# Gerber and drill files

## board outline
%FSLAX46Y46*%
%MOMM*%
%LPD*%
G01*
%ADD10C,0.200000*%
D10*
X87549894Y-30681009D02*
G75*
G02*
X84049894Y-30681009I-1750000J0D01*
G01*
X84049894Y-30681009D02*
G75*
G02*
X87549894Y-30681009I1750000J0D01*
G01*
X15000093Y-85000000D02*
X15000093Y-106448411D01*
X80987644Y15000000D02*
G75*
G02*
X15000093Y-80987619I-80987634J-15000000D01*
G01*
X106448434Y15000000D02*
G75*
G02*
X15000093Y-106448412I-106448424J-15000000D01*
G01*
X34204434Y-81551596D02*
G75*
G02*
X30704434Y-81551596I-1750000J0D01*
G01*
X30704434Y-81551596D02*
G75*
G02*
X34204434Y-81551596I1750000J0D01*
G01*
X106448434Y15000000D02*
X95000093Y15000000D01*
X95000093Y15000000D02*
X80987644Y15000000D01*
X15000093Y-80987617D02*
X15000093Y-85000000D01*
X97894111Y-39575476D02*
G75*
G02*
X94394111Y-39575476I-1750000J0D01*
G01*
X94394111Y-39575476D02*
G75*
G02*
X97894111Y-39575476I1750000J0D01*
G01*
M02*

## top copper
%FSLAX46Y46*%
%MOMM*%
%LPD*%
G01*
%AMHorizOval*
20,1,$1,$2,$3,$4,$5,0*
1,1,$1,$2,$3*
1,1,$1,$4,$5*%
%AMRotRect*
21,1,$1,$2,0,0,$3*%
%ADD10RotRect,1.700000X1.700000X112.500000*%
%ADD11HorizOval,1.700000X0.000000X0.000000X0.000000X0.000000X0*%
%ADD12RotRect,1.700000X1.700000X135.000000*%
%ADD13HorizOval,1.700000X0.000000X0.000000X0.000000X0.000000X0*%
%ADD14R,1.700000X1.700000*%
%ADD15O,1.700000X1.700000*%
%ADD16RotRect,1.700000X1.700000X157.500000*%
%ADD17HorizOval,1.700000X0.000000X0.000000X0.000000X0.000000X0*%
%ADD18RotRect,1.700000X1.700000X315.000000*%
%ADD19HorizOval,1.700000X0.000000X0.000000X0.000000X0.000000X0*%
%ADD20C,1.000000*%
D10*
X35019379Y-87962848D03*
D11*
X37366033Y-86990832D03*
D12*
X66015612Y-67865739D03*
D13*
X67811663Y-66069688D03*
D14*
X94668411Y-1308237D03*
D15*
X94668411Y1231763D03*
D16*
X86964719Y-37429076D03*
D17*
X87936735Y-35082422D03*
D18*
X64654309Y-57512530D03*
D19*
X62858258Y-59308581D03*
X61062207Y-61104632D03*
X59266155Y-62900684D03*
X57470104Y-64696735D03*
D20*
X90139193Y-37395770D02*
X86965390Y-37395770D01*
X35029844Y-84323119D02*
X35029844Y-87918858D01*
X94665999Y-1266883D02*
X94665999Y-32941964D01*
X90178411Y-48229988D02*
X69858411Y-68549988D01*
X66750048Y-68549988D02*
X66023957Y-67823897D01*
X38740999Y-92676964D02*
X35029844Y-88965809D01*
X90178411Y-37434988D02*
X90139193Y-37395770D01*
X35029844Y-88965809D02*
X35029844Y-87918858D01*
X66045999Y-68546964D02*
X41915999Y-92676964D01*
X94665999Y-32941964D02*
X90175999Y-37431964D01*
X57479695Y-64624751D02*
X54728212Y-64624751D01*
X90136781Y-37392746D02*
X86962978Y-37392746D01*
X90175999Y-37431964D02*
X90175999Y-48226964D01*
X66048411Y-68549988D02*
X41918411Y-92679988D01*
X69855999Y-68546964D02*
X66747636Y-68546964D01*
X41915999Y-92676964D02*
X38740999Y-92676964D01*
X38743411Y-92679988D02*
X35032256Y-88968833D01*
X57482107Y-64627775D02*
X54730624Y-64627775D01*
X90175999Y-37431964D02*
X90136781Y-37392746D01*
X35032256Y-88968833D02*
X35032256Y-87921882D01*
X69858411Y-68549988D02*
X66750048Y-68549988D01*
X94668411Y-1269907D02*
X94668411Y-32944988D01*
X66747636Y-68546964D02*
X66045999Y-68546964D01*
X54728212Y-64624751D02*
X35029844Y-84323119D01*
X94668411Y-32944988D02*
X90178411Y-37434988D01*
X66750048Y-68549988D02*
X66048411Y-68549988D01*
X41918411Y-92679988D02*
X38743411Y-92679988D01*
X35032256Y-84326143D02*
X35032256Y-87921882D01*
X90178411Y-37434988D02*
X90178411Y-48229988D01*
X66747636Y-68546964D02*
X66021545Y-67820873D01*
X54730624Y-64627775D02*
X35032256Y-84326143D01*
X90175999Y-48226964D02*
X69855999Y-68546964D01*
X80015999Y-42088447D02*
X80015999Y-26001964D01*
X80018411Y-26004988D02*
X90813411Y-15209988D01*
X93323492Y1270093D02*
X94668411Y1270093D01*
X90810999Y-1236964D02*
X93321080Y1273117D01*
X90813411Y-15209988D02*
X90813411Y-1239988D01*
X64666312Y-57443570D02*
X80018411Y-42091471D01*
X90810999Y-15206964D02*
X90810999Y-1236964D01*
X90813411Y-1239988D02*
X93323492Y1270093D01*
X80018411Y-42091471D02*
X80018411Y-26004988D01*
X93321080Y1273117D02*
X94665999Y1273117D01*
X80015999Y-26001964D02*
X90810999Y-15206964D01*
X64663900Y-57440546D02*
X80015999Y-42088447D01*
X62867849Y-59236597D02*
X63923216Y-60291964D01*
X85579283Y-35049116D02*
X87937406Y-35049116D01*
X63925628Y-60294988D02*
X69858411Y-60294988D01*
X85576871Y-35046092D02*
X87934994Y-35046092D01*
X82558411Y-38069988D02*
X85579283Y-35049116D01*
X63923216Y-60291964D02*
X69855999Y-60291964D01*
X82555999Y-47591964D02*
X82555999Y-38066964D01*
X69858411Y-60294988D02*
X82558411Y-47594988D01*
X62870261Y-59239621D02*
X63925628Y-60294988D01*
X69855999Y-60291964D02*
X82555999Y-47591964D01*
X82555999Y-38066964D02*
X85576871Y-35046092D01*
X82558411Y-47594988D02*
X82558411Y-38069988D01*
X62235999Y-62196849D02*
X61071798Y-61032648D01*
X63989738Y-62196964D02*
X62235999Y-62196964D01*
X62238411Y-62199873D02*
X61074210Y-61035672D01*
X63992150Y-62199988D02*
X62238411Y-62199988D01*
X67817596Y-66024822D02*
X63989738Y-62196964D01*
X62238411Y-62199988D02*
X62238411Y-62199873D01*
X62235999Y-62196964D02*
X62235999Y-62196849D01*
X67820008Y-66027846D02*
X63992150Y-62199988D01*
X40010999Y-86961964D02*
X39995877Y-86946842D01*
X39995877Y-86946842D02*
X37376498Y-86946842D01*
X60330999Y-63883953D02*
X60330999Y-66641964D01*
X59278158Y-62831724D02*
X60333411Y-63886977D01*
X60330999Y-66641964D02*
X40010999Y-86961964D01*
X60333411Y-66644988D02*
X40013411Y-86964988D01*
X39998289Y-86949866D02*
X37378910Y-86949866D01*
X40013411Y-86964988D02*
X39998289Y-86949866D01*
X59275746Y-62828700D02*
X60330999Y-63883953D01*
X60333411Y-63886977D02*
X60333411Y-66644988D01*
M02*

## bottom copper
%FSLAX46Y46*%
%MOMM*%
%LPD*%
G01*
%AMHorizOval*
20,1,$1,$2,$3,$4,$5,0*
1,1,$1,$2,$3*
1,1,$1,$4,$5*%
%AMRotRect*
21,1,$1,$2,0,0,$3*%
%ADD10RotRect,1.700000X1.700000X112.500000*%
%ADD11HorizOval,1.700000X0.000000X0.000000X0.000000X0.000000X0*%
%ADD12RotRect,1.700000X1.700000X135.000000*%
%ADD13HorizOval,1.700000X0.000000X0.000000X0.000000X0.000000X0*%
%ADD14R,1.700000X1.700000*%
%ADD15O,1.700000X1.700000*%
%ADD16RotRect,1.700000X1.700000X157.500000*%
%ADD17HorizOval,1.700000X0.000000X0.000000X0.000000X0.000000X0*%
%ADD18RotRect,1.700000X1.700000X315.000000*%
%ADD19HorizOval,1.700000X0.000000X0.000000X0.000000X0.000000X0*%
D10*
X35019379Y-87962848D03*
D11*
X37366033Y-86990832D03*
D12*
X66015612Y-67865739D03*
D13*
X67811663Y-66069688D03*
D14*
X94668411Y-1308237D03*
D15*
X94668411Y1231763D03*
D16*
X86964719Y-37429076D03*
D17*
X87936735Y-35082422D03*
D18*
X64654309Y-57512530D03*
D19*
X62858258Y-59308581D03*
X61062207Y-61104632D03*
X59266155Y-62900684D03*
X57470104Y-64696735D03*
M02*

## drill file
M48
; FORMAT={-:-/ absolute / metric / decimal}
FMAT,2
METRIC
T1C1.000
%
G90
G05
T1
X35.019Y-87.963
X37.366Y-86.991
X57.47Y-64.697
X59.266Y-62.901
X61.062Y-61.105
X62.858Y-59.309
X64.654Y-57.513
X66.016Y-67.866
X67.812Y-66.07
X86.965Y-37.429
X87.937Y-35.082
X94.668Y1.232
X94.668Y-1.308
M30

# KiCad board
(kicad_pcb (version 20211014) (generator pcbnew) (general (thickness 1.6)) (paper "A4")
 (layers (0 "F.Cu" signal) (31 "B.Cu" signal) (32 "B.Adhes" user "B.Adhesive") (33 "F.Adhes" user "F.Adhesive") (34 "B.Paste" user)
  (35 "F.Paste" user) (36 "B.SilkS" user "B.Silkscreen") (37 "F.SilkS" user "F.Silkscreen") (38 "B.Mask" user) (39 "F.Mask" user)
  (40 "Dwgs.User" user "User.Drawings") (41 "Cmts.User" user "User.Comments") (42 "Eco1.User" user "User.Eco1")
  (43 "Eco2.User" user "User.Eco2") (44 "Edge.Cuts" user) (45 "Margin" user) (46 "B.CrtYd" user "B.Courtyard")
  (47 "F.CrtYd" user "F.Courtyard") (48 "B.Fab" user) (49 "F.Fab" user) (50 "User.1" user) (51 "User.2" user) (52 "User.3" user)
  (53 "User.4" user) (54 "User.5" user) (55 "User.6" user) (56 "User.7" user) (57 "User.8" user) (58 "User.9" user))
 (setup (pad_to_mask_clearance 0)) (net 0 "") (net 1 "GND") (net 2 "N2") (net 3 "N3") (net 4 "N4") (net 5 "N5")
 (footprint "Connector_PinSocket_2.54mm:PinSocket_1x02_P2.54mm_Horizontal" (layer "F.Cu") (at 35.019379 87.962848 112.5)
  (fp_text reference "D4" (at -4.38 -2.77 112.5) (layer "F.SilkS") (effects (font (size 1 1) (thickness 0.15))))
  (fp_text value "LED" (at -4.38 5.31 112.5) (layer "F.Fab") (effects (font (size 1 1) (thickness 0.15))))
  (pad "1" thru_hole rect (at 0 0 112.5) (size 1.7 1.7) (drill 1) (layers *.Cu *.Mask) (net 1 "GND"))
  (pad "2" thru_hole oval (at 0 2.54 112.5) (size 1.7 1.7) (drill 1) (layers *.Cu *.Mask) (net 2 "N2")))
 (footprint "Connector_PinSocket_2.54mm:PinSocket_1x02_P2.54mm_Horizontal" (layer "F.Cu") (at 66.015612 67.865739 135)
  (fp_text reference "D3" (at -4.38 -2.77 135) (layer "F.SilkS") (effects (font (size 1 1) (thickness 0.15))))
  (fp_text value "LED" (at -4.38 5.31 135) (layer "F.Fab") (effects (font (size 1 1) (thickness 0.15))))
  (pad "1" thru_hole rect (at 0 0 135) (size 1.7 1.7) (drill 1) (layers *.Cu *.Mask) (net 1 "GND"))
  (pad "2" thru_hole oval (at 0 2.54 135) (size 1.7 1.7) (drill 1) (layers *.Cu *.Mask) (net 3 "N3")))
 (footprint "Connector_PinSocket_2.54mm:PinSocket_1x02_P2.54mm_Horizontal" (layer "F.Cu") (at 94.668411 1.308237 180)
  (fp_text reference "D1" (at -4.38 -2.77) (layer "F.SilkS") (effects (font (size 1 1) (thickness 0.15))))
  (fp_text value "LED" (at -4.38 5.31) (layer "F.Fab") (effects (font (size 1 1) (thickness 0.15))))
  (pad "1" thru_hole rect (at 0 0 180) (size 1.7 1.7) (drill 1) (layers *.Cu *.Mask) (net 1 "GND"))
  (pad "2" thru_hole oval (at 0 2.54 180) (size 1.7 1.7) (drill 1) (layers *.Cu *.Mask) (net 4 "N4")))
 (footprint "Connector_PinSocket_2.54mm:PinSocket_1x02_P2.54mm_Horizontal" (layer "F.Cu") (at 86.964719 37.429076 157.5)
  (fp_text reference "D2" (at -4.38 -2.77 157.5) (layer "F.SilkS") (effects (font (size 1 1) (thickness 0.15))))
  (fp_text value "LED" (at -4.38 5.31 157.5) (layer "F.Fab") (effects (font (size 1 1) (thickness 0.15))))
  (pad "1" thru_hole rect (at 0 0 157.5) (size 1.7 1.7) (drill 1) (layers *.Cu *.Mask) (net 1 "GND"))
  (pad "2" thru_hole oval (at 0 2.54 157.5) (size 1.7 1.7) (drill 1) (layers *.Cu *.Mask) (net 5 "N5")))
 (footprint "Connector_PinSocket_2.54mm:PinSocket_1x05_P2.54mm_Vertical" (layer "F.Cu") (at 64.654309 57.51253 -45)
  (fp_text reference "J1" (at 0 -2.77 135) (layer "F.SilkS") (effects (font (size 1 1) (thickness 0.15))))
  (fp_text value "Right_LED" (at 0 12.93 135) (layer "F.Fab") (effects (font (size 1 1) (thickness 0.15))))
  (pad "1" thru_hole rect (at 0 0 315) (size 1.7 1.7) (drill 1) (layers *.Cu *.Mask) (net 4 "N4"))
  (pad "2" thru_hole oval (at 0 2.54 315) (size 1.7 1.7) (drill 1) (layers *.Cu *.Mask) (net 5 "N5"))
  (pad "3" thru_hole oval (at 0 5.08 315) (size 1.7 1.7) (drill 1) (layers *.Cu *.Mask) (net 3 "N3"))
  (pad "4" thru_hole oval (at 0 7.62 315) (size 1.7 1.7) (drill 1) (layers *.Cu *.Mask) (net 2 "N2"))
  (pad "5" thru_hole oval (at 0 10.16 315) (size 1.7 1.7) (drill 1) (layers *.Cu *.Mask) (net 1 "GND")))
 (gr_circle (center 85.799894 30.681009) (end 87.549894 30.681009) (layer "Edge.Cuts") (width 0.2) (fill none))
 (gr_line (start 15.000093 85) (end 15.000093 106.448411) (layer "Edge.Cuts") (width 0.2))
 (gr_arc (start 80.987644 -15) (mid 67.873541 46.660268) (end 15.000093 80.987617) (layer "Edge.Cuts") (width 0.2))
 (gr_arc (start 106.448434 -15) (mid 85.877039 64.663767) (end 15.000093 106.448411) (layer "Edge.Cuts") (width 0.2))
 (gr_circle (center 32.454434 81.551596) (end 34.204434 81.551596) (layer "Edge.Cuts") (width 0.2) (fill none))
 (gr_line (start 106.448434 -15) (end 95.000093 -15) (layer "Edge.Cuts") (width 0.2))
 (gr_line (start 95.000093 -15) (end 80.987644 -15) (layer "Edge.Cuts") (width 0.2))
 (gr_line (start 15.000093 80.987617) (end 15.000093 85) (layer "Edge.Cuts") (width 0.2))
 (gr_circle (center 96.144111 39.575476) (end 97.894111 39.575476) (layer "Edge.Cuts") (width 0.2) (fill none))
 (segment (start 90.139193 37.39577) (end 86.96539 37.39577) (width 1) (layer "F.Cu") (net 1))
 (segment (start 35.029844 84.323119) (end 35.029844 87.918858) (width 1) (layer "F.Cu") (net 1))
 (segment (start 94.665999 1.266883) (end 94.665999 32.941964) (width 1) (layer "F.Cu") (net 1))
 (segment (start 90.178411 48.229988) (end 69.858411 68.549988) (width 1) (layer "F.Cu") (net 1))
 (segment (start 66.750048 68.549988) (end 66.023957 67.823897) (width 1) (layer "F.Cu") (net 1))
 (segment (start 38.740999 92.676964) (end 35.029844 88.965809) (width 1) (layer "F.Cu") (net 1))
 (segment (start 90.178411 37.434988) (end 90.139193 37.39577) (width 1) (layer "F.Cu") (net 1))
 (segment (start 35.029844 88.965809) (end 35.029844 87.918858) (width 1) (layer "F.Cu") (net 1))
 (segment (start 66.045999 68.546964) (end 41.915999 92.676964) (width 1) (layer "F.Cu") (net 1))
 (segment (start 94.665999 32.941964) (end 90.175999 37.431964) (width 1) (layer "F.Cu") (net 1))
 (segment (start 57.479695 64.624751) (end 54.728212 64.624751) (width 1) (layer "F.Cu") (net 1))
 (segment (start 90.136781 37.392746) (end 86.962978 37.392746) (width 1) (layer "F.Cu") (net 1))
 (segment (start 90.175999 37.431964) (end 90.175999 48.226964) (width 1) (layer "F.Cu") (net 1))
 (segment (start 66.048411 68.549988) (end 41.918411 92.679988) (width 1) (layer "F.Cu") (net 1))
 (segment (start 69.855999 68.546964) (end 66.747636 68.546964) (width 1) (layer "F.Cu") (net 1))
 (segment (start 41.915999 92.676964) (end 38.740999 92.676964) (width 1) (layer "F.Cu") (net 1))
 (segment (start 38.743411 92.679988) (end 35.032256 88.968833) (width 1) (layer "F.Cu") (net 1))
 (segment (start 57.482107 64.627775) (end 54.730624 64.627775) (width 1) (layer "F.Cu") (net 1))
 (segment (start 90.175999 37.431964) (end 90.136781 37.392746) (width 1) (layer "F.Cu") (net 1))
 (segment (start 35.032256 88.968833) (end 35.032256 87.921882) (width 1) (layer "F.Cu") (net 1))
 (segment (start 69.858411 68.549988) (end 66.750048 68.549988) (width 1) (layer "F.Cu") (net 1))
 (segment (start 94.668411 1.269907) (end 94.668411 32.944988) (width 1) (layer "F.Cu") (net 1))
 (segment (start 66.747636 68.546964) (end 66.045999 68.546964) (width 1) (layer "F.Cu") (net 1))
 (segment (start 54.728212 64.624751) (end 35.029844 84.323119) (width 1) (layer "F.Cu") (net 1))
 (segment (start 94.668411 32.944988) (end 90.178411 37.434988) (width 1) (layer "F.Cu") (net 1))
 (segment (start 66.750048 68.549988) (end 66.048411 68.549988) (width 1) (layer "F.Cu") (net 1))
 (segment (start 41.918411 92.679988) (end 38.743411 92.679988) (width 1) (layer "F.Cu") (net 1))
 (segment (start 35.032256 84.326143) (end 35.032256 87.921882) (width 1) (layer "F.Cu") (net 1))
 (segment (start 90.178411 37.434988) (end 90.178411 48.229988) (width 1) (layer "F.Cu") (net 1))
 (segment (start 66.747636 68.546964) (end 66.021545 67.820873) (width 1) (layer "F.Cu") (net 1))
 (segment (start 54.730624 64.627775) (end 35.032256 84.326143) (width 1) (layer "F.Cu") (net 1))
 (segment (start 90.175999 48.226964) (end 69.855999 68.546964) (width 1) (layer "F.Cu") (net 1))
 (segment (start 80.015999 42.088447) (end 80.015999 26.001964) (width 1) (layer "F.Cu") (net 4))
 (segment (start 80.018411 26.004988) (end 90.813411 15.209988) (width 1) (layer "F.Cu") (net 4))
 (segment (start 93.323492 -1.270093) (end 94.668411 -1.270093) (width 1) (layer "F.Cu") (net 4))
 (segment (start 90.810999 1.236964) (end 93.32108 -1.273117) (width 1) (layer "F.Cu") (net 4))
 (segment (start 90.813411 15.209988) (end 90.813411 1.239988) (width 1) (layer "F.Cu") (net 4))
 (segment (start 64.666312 57.44357) (end 80.018411 42.091471) (width 1) (layer "F.Cu") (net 4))
 (segment (start 90.810999 15.206964) (end 90.810999 1.236964) (width 1) (layer "F.Cu") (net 4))
 (segment (start 90.813411 1.239988) (end 93.323492 -1.270093) (width 1) (layer "F.Cu") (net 4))
 (segment (start 80.018411 42.091471) (end 80.018411 26.004988) (width 1) (layer "F.Cu") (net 4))
 (segment (start 93.32108 -1.273117) (end 94.665999 -1.273117) (width 1) (layer "F.Cu") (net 4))
 (segment (start 80.015999 26.001964) (end 90.810999 15.206964) (width 1) (layer "F.Cu") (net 4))
 (segment (start 64.6639 57.440546) (end 80.015999 42.088447) (width 1) (layer "F.Cu") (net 4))
 (segment (start 62.867849 59.236597) (end 63.923216 60.291964) (width 1) (layer "F.Cu") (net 5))
 (segment (start 85.579283 35.049116) (end 87.937406 35.049116) (width 1) (layer "F.Cu") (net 5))
 (segment (start 63.925628 60.294988) (end 69.858411 60.294988) (width 1) (layer "F.Cu") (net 5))
 (segment (start 85.576871 35.046092) (end 87.934994 35.046092) (width 1) (layer "F.Cu") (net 5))
 (segment (start 82.558411 38.069988) (end 85.579283 35.049116) (width 1) (layer "F.Cu") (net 5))
 (segment (start 63.923216 60.291964) (end 69.855999 60.291964) (width 1) (layer "F.Cu") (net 5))
 (segment (start 82.555999 47.591964) (end 82.555999 38.066964) (width 1) (layer "F.Cu") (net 5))
 (segment (start 69.858411 60.294988) (end 82.558411 47.594988) (width 1) (layer "F.Cu") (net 5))
 (segment (start 62.870261 59.239621) (end 63.925628 60.294988) (width 1) (layer "F.Cu") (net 5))
 (segment (start 69.855999 60.291964) (end 82.555999 47.591964) (width 1) (layer "F.Cu") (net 5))
 (segment (start 82.555999 38.066964) (end 85.576871 35.046092) (width 1) (layer "F.Cu") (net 5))
 (segment (start 82.558411 47.594988) (end 82.558411 38.069988) (width 1) (layer "F.Cu") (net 5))
 (segment (start 62.235999 62.196849) (end 61.071798 61.032648) (width 1) (layer "F.Cu") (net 3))
 (segment (start 63.989738 62.196964) (end 62.235999 62.196964) (width 1) (layer "F.Cu") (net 3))
 (segment (start 62.238411 62.199873) (end 61.07421 61.035672) (width 1) (layer "F.Cu") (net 3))
 (segment (start 63.99215 62.199988) (end 62.238411 62.199988) (width 1) (layer "F.Cu") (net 3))
 (segment (start 67.817596 66.024822) (end 63.989738 62.196964) (width 1) (layer "F.Cu") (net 3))
 (segment (start 62.238411 62.199988) (end 62.238411 62.199873) (width 1) (layer "F.Cu") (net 3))
 (segment (start 62.235999 62.196964) (end 62.235999 62.196849) (width 1) (layer "F.Cu") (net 3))
 (segment (start 67.820008 66.027846) (end 63.99215 62.199988) (width 1) (layer "F.Cu") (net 3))
 (segment (start 40.010999 86.961964) (end 39.995877 86.946842) (width 1) (layer "F.Cu") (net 2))
 (segment (start 39.995877 86.946842) (end 37.376498 86.946842) (width 1) (layer "F.Cu") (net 2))
 (segment (start 60.330999 63.883953) (end 60.330999 66.641964) (width 1) (layer "F.Cu") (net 2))
 (segment (start 59.278158 62.831724) (end 60.333411 63.886977) (width 1) (layer "F.Cu") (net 2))
 (segment (start 60.330999 66.641964) (end 40.010999 86.961964) (width 1) (layer "F.Cu") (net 2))
 (segment (start 60.333411 66.644988) (end 40.013411 86.964988) (width 1) (layer "F.Cu") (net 2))
 (segment (start 39.998289 86.949866) (end 37.37891 86.949866) (width 1) (layer "F.Cu") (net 2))
 (segment (start 40.013411 86.964988) (end 39.998289 86.949866) (width 1) (layer "F.Cu") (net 2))
 (segment (start 59.275746 62.8287) (end 60.330999 63.883953) (width 1) (layer "F.Cu") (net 2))
 (segment (start 60.333411 63.886977) (end 60.333411 66.644988) (width 1) (layer "F.Cu") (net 2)))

